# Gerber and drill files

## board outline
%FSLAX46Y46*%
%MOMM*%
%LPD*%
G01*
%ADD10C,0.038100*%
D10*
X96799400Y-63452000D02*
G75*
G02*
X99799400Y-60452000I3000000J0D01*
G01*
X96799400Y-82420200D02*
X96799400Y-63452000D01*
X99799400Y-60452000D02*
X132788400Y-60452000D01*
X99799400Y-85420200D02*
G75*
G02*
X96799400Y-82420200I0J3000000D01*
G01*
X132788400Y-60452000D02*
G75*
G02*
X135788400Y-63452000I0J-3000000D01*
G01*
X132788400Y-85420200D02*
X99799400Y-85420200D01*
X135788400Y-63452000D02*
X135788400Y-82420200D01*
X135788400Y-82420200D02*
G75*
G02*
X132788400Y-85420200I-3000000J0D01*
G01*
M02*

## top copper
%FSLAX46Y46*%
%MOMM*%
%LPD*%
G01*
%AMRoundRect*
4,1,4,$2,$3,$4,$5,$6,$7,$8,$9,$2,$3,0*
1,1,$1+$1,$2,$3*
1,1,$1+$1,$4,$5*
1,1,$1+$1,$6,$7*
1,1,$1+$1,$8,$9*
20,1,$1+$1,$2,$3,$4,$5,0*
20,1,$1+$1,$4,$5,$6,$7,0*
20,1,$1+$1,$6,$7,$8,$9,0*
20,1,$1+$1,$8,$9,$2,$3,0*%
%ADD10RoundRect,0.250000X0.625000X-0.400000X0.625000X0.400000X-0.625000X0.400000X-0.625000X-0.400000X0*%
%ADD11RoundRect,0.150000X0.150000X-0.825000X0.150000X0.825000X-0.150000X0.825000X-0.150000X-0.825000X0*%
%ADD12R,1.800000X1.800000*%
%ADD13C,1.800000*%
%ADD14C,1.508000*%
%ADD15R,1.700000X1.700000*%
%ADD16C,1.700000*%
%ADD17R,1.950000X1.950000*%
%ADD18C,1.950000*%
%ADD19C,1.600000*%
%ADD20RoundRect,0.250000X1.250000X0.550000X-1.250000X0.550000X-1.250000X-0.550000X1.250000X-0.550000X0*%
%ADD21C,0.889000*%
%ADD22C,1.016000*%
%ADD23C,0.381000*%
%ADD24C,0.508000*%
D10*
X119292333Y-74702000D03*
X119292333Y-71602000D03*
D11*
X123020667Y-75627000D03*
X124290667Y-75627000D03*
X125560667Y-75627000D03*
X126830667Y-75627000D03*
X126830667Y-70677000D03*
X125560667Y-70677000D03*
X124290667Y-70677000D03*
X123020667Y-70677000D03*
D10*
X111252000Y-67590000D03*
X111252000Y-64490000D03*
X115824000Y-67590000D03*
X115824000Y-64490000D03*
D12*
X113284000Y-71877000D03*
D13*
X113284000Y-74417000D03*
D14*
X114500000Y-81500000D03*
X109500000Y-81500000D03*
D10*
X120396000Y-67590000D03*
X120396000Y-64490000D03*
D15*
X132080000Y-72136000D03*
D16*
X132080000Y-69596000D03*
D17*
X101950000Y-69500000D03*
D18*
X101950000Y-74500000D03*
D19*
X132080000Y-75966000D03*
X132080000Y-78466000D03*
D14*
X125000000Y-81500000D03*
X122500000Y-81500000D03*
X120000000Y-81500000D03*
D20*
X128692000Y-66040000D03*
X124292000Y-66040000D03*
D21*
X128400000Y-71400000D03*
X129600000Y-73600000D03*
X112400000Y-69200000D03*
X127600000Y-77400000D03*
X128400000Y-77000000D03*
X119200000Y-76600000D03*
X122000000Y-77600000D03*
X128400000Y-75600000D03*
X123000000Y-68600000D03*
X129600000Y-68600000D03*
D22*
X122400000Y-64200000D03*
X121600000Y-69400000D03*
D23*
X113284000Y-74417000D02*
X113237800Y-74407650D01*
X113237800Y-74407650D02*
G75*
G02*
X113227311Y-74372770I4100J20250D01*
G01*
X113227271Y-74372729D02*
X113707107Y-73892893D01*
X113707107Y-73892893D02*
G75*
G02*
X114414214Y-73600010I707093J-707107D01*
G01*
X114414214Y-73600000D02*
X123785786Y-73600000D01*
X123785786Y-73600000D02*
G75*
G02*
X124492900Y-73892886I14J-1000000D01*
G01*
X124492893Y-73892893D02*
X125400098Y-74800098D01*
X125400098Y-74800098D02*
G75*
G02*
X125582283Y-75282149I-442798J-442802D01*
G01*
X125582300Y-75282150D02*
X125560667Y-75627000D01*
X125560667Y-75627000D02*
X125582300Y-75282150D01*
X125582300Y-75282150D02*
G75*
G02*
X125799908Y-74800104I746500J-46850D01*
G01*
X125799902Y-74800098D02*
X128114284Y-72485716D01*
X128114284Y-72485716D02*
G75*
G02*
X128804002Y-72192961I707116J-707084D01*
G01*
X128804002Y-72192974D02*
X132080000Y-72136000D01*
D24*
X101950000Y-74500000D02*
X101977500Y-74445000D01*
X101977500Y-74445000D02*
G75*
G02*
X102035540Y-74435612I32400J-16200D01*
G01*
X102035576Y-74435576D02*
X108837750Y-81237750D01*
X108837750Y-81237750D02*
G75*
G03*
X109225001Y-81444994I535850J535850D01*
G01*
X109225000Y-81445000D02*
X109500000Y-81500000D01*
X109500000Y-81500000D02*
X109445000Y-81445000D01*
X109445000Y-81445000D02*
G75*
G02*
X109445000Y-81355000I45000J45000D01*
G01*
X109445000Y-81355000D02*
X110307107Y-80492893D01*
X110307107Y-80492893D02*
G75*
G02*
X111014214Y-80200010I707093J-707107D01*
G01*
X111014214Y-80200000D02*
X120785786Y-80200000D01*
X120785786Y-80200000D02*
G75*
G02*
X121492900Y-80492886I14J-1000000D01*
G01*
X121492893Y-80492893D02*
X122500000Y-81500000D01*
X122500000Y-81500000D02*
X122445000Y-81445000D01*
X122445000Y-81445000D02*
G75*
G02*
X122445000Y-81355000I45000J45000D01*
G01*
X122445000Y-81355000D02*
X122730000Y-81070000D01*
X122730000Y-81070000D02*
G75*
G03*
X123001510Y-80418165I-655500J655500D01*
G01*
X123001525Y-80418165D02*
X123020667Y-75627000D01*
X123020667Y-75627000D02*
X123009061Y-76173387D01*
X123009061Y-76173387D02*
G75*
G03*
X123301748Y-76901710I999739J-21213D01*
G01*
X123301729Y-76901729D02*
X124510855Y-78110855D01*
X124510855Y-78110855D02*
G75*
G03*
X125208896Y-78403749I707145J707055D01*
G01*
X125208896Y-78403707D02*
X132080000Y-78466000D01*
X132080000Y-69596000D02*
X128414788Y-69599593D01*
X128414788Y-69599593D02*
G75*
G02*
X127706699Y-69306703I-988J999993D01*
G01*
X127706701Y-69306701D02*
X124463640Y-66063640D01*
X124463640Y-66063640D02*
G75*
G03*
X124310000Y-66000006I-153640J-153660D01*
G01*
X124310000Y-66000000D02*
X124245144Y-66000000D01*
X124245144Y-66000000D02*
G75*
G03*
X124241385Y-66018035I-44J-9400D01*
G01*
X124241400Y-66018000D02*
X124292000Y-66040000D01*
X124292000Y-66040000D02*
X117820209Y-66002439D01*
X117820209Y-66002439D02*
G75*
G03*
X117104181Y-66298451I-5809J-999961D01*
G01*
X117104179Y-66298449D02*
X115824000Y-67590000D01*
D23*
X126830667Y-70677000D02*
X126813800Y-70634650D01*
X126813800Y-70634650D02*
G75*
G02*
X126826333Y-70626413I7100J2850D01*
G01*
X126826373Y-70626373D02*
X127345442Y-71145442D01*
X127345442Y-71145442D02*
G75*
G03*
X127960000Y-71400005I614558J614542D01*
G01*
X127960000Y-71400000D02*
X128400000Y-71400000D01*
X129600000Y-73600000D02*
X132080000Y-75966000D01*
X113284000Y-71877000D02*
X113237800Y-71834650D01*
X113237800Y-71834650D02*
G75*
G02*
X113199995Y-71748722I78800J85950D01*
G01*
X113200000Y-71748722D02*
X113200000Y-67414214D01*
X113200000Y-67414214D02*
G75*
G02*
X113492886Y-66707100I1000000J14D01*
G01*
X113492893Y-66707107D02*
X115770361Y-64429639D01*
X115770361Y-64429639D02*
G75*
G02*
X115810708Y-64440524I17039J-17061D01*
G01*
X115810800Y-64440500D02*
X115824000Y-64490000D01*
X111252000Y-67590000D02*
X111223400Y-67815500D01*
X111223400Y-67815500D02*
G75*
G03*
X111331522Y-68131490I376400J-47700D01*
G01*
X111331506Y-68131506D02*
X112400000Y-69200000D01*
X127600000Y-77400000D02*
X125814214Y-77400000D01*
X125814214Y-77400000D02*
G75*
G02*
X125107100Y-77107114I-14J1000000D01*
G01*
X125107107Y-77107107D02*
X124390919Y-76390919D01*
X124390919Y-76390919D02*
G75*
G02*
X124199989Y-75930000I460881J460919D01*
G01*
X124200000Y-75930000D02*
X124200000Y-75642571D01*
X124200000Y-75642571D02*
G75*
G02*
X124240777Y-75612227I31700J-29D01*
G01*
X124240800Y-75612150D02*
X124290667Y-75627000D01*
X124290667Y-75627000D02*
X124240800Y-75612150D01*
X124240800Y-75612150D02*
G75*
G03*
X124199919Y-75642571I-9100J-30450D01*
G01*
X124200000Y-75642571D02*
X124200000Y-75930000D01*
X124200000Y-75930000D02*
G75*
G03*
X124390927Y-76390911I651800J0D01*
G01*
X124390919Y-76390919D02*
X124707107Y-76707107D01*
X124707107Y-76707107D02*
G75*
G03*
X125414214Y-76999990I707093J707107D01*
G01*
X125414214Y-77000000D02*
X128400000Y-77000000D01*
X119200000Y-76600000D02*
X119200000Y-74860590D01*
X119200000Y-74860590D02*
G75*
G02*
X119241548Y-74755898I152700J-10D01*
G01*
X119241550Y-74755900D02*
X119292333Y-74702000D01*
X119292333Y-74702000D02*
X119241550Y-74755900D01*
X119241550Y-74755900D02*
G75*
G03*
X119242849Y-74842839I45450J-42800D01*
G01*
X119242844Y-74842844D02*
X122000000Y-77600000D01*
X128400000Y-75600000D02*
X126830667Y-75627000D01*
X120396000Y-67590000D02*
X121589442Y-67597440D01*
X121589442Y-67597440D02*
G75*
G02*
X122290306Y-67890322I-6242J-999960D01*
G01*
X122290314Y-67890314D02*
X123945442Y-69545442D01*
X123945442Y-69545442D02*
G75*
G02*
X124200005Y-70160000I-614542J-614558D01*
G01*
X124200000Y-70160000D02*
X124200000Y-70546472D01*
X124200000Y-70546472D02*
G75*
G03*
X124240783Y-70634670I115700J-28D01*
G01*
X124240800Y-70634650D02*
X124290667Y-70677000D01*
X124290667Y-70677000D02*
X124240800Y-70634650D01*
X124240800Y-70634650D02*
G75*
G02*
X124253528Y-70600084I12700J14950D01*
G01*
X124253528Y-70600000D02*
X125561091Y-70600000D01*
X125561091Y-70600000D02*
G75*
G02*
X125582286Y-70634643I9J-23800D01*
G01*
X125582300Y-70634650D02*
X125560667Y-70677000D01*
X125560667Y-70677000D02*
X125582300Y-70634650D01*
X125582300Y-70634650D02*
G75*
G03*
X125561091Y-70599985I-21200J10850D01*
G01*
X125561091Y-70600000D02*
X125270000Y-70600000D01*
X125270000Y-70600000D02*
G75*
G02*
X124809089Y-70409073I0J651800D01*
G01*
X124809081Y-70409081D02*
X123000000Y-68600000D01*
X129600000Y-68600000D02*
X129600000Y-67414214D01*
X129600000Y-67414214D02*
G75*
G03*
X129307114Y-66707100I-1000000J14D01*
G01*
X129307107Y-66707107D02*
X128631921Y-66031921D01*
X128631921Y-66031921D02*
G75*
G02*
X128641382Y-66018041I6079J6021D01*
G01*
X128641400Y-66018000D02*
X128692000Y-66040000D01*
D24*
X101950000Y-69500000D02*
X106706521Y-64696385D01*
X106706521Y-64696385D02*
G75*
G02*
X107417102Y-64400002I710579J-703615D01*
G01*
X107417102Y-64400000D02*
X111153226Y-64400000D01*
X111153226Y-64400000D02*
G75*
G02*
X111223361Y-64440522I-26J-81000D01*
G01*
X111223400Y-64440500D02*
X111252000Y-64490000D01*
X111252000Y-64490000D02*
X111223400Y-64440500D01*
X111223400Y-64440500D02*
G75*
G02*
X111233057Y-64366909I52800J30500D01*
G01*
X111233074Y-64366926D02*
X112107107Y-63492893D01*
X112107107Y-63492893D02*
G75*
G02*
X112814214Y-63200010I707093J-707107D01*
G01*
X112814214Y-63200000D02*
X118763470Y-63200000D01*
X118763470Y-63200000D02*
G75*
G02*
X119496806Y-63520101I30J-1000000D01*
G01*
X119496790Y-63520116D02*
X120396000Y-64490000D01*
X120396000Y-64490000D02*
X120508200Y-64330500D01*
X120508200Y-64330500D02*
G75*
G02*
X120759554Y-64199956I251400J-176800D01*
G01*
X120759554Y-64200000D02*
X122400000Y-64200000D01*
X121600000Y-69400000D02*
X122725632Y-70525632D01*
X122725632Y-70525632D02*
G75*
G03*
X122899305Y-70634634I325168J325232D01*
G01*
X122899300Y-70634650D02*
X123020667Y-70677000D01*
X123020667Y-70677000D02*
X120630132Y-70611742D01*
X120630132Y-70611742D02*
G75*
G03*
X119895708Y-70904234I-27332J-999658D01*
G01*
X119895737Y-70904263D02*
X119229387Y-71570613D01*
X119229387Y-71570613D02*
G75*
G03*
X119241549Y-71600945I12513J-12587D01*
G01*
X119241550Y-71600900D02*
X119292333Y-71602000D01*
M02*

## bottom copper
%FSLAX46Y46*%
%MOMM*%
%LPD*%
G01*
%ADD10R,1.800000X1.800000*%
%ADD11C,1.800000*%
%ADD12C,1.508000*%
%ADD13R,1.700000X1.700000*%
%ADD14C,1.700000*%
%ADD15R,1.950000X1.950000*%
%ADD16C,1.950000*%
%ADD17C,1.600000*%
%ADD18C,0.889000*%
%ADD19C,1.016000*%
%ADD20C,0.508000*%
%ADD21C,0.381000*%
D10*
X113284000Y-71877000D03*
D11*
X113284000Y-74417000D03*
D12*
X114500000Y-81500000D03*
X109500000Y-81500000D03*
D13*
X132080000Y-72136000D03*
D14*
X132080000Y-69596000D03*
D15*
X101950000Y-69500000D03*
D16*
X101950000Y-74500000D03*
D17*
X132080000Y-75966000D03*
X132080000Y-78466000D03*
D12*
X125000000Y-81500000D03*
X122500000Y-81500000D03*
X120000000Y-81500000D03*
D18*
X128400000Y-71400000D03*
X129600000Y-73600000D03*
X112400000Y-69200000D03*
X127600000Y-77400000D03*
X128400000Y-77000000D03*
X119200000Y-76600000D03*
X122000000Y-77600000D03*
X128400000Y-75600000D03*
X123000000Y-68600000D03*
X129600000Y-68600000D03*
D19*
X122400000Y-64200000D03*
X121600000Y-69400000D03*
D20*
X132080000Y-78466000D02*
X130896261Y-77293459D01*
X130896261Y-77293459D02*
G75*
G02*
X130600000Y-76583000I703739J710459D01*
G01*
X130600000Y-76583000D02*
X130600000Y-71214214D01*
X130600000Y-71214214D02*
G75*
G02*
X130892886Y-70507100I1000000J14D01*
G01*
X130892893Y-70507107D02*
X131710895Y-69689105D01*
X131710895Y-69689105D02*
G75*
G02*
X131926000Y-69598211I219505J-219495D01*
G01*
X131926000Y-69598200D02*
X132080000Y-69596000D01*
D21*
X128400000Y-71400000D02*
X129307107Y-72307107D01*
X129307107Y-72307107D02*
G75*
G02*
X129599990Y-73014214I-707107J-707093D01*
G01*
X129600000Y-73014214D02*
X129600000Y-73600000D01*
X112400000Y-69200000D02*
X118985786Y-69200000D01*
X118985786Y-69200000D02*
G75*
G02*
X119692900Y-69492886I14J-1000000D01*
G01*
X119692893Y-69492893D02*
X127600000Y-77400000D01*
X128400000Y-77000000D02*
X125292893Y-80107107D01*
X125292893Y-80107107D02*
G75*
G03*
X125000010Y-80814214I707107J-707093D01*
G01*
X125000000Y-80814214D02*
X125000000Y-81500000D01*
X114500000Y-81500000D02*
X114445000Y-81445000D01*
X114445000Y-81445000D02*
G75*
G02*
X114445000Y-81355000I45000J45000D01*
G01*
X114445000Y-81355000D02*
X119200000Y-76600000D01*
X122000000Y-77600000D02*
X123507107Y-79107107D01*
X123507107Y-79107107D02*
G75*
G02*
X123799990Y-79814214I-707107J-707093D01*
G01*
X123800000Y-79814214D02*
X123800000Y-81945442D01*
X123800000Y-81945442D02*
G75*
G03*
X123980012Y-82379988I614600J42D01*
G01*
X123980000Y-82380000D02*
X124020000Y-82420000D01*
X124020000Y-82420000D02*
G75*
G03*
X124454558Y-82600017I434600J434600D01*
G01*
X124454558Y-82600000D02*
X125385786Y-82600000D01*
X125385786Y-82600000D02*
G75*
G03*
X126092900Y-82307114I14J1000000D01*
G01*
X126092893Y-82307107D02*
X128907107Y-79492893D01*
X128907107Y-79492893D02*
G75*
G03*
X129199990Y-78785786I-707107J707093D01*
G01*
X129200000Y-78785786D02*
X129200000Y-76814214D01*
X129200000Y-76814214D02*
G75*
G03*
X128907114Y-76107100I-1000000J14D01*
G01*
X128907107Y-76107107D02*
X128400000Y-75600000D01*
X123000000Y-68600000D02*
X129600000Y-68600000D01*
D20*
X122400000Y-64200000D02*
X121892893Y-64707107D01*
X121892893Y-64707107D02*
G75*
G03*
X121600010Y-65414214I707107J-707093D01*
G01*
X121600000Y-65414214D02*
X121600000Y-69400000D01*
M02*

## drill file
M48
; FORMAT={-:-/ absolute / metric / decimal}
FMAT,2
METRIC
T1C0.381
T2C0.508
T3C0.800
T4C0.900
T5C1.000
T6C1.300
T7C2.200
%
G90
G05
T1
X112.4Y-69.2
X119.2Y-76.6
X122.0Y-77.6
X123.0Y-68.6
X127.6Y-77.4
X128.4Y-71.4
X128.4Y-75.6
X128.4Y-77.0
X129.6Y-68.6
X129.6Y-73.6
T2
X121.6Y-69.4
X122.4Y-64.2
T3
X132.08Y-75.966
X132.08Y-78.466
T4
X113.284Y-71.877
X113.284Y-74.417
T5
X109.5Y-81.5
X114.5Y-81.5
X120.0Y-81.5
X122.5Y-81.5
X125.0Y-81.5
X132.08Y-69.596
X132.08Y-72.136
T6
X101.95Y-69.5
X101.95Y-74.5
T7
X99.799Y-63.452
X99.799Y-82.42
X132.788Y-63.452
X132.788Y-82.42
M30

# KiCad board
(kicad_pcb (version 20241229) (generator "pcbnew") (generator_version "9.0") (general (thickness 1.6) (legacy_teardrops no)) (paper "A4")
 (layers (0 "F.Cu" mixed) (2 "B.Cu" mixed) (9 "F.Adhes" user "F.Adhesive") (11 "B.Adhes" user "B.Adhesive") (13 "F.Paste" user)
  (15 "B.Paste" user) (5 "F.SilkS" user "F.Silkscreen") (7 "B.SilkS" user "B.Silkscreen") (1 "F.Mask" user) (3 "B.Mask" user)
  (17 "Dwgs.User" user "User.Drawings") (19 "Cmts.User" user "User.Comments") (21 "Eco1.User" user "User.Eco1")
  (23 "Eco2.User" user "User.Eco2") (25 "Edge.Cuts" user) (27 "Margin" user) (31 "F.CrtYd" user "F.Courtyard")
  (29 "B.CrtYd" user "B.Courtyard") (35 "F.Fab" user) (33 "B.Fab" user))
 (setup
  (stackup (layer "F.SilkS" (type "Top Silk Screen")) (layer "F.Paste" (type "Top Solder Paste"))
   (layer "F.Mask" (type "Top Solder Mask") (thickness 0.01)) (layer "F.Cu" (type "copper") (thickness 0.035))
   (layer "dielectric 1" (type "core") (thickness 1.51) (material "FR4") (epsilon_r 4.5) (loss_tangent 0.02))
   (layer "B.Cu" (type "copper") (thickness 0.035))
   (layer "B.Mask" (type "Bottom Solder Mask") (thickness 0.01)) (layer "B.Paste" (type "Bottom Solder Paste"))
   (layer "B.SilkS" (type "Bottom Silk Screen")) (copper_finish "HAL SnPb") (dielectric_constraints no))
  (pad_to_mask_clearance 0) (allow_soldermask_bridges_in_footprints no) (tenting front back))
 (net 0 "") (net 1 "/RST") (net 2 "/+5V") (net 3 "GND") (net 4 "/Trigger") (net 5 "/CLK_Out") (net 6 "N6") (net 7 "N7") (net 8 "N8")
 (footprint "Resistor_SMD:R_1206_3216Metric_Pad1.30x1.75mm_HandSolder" (layer "F.Cu") (at 119.292333 73.152 90)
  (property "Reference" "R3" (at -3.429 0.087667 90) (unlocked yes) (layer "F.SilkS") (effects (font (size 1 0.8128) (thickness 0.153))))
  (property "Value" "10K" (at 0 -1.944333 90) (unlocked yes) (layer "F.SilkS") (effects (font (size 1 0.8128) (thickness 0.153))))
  (pad "1" smd roundrect (at -1.55 0 90) (size 1.3 1.75) (layers "F.Cu" "F.Mask" "F.Paste") (roundrect_rratio 0.192308) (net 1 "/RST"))
  (pad "2" smd roundrect (at 1.55 0 90) (size 1.3 1.75) (layers "F.Cu" "F.Mask" "F.Paste") (roundrect_rratio 0.192308) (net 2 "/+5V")))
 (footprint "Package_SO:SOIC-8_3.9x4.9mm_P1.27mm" (layer "F.Cu") (at 124.925667 73.152 90)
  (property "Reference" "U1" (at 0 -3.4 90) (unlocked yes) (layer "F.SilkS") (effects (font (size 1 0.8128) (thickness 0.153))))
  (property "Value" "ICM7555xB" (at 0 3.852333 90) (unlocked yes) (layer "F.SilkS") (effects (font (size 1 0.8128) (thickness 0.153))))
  (pad "1" smd roundrect (at -2.475 -1.905 90) (size 1.95 0.6) (layers "F.Cu" "F.Mask" "F.Paste") (roundrect_rratio 0.25) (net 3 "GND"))
  (pad "2" smd roundrect (at -2.475 -0.635 90) (size 1.95 0.6) (layers "F.Cu" "F.Mask" "F.Paste") (roundrect_rratio 0.25) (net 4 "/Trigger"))
  (pad "3" smd roundrect (at -2.475 0.635 90) (size 1.95 0.6) (layers "F.Cu" "F.Mask" "F.Paste") (roundrect_rratio 0.25) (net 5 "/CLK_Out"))
  (pad "4" smd roundrect (at -2.475 1.905 90) (size 1.95 0.6) (layers "F.Cu" "F.Mask" "F.Paste") (roundrect_rratio 0.25) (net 1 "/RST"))
  (pad "5" smd roundrect (at 2.475 1.905 90) (size 1.95 0.6) (layers "F.Cu" "F.Mask" "F.Paste") (roundrect_rratio 0.25) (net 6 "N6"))
  (pad "6" smd roundrect (at 2.475 0.635 90) (size 1.95 0.6) (layers "F.Cu" "F.Mask" "F.Paste") (roundrect_rratio 0.25) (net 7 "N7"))
  (pad "7" smd roundrect (at 2.475 -0.635 90) (size 1.95 0.6) (layers "F.Cu" "F.Mask" "F.Paste") (roundrect_rratio 0.25) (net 7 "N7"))
  (pad "8" smd roundrect (at 2.475 -1.905 90) (size 1.95 0.6) (layers "F.Cu" "F.Mask" "F.Paste") (roundrect_rratio 0.25) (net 2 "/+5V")))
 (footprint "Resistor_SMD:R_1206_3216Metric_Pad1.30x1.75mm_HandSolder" (layer "F.Cu") (at 111.252 66.04 90)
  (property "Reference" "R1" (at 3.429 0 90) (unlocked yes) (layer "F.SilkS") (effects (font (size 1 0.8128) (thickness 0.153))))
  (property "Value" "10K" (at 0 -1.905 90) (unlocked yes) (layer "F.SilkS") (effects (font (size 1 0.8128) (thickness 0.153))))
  (pad "1" smd roundrect (at -1.55 0 90) (size 1.3 1.75) (layers "F.Cu" "F.Mask" "F.Paste") (roundrect_rratio 0.192308) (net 4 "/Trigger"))
  (pad "2" smd roundrect (at 1.55 0 90) (size 1.3 1.75) (layers "F.Cu" "F.Mask" "F.Paste") (roundrect_rratio 0.192308) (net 2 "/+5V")))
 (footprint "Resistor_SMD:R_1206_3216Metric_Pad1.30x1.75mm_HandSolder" (layer "F.Cu") (at 115.824 66.04 90)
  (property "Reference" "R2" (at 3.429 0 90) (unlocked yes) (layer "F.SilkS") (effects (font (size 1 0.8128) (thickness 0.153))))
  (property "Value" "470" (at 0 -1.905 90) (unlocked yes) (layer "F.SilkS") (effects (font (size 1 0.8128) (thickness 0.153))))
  (pad "1" smd roundrect (at -1.55 0 90) (size 1.3 1.75) (layers "F.Cu" "F.Mask" "F.Paste") (roundrect_rratio 0.192308) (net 3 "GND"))
  (pad "2" smd roundrect (at 1.55 0 90) (size 1.3 1.75) (layers "F.Cu" "F.Mask" "F.Paste") (roundrect_rratio 0.192308) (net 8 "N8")))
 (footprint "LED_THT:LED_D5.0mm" (layer "F.Cu") (at 113.284 71.877 -90)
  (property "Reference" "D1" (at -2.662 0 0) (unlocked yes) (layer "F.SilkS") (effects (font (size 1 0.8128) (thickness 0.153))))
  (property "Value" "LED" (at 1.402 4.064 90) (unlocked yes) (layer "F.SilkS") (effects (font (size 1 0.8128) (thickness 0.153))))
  (pad "1" thru_hole rect (at 0 0 270) (size 1.8 1.8) (drill 0.9) (layers "*.Cu" "*.Mask") (remove_unused_layers no) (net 8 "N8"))
  (pad "2" thru_hole circle (at 2.54 0 270) (size 1.8 1.8) (drill 0.9) (layers "*.Cu" "*.Mask") (remove_unused_layers no) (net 5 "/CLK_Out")))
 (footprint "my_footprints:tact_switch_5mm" (layer "F.Cu") (at 112 81.5 180)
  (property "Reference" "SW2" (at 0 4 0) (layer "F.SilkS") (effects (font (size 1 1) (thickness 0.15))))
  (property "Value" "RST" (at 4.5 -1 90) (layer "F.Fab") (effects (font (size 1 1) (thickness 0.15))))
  (pad "1" thru_hole circle (at -2.5 0 180) (size 1.508 1.508) (drill 1) (layers "*.Cu" "*.Mask") (remove_unused_layers no) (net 1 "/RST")
   (solder_mask_margin 0.102))
  (pad "2" thru_hole circle (at 2.5 0 180) (size 1.508 1.508) (drill 1) (layers "*.Cu" "*.Mask") (remove_unused_layers no) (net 3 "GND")
   (solder_mask_margin 0.102)))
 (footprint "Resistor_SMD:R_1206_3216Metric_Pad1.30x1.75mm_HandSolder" (layer "F.Cu") (at 120.396 66.04 90)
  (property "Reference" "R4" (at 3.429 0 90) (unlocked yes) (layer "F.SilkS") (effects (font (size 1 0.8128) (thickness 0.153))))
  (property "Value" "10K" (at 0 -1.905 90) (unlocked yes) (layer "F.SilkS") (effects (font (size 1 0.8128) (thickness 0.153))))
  (pad "1" smd roundrect (at -1.55 0 90) (size 1.3 1.75) (layers "F.Cu" "F.Mask" "F.Paste") (roundrect_rratio 0.192308) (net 7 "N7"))
  (pad "2" smd roundrect (at 1.55 0 90) (size 1.3 1.75) (layers "F.Cu" "F.Mask" "F.Paste") (roundrect_rratio 0.192308) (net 2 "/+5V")))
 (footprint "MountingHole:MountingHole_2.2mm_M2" (layer "F.Cu") (at 99.7994 63.452)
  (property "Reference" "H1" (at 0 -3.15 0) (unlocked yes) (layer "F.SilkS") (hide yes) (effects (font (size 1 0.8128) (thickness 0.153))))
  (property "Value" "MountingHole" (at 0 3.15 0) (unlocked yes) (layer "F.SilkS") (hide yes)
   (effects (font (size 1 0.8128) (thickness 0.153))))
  (pad "" np_thru_hole circle (at 0 0) (size 2.2 2.2) (drill 2.2) (layers "*.Cu" "*.Mask")))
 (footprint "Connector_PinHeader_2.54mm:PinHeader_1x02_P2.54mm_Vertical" (layer "F.Cu") (at 132.08 72.136 180)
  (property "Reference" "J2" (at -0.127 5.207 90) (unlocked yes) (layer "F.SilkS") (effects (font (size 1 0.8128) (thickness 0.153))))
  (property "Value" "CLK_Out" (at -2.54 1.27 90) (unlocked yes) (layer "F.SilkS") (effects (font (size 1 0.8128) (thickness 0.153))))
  (pad "1" thru_hole rect (at 0 0 180) (size 1.7 1.7) (drill 1) (layers "*.Cu" "*.Mask") (remove_unused_layers no) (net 5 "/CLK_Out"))
  (pad "2" thru_hole circle (at 0 2.54 180) (size 1.7 1.7) (drill 1) (layers "*.Cu" "*.Mask") (remove_unused_layers no) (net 3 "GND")))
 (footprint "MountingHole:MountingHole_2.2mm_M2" (layer "F.Cu") (at 132.7884 82.4202)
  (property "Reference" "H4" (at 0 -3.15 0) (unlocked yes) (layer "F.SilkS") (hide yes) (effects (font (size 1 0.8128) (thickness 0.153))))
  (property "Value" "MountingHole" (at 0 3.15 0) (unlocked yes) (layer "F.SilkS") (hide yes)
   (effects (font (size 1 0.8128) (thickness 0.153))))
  (pad "" np_thru_hole circle (at 0 0) (size 2.2 2.2) (drill 2.2) (layers "*.Cu" "*.Mask")))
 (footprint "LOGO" (layer "F.Cu") (at 105.5 63.5)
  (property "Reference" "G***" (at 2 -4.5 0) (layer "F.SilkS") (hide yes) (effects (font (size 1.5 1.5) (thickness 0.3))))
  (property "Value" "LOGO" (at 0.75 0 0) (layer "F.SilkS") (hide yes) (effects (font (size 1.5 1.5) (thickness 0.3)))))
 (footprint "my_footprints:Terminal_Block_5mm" (layer "F.Cu") (at 101.95 72 -90)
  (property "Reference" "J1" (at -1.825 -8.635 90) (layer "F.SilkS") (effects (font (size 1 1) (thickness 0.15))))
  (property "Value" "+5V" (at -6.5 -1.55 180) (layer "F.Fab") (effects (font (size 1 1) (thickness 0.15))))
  (pad "1" thru_hole rect (at -2.5 0 270) (size 1.95 1.95) (drill 1.3) (layers "*.Cu" "*.Mask") (remove_unused_layers no) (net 2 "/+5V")
   (solder_mask_margin 0.102))
  (pad "2" thru_hole circle (at 2.5 0 270) (size 1.95 1.95) (drill 1.3) (layers "*.Cu" "*.Mask") (remove_unused_layers no) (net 3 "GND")
   (solder_mask_margin 0.102)))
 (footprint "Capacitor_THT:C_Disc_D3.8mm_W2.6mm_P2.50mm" (layer "F.Cu") (at 132.08 75.966 -90)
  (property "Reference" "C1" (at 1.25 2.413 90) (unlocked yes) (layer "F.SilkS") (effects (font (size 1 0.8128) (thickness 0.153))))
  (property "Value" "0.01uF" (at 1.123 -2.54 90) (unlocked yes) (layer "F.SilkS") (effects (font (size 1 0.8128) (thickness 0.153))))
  (pad "1" thru_hole circle (at 0 0 270) (size 1.6 1.6) (drill 0.8) (layers "*.Cu" "*.Mask") (remove_unused_layers no) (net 6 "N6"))
  (pad "2" thru_hole circle (at 2.5 0 270) (size 1.6 1.6) (drill 0.8) (layers "*.Cu" "*.Mask") (remove_unused_layers no) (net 3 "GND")))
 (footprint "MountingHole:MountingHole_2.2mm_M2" (layer "F.Cu") (at 132.7884 63.452)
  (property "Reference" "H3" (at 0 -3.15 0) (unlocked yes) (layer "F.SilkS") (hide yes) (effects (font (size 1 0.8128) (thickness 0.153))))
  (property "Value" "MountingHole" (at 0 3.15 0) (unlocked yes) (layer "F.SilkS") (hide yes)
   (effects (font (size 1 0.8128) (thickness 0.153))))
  (pad "" np_thru_hole circle (at 0 0) (size 2.2 2.2) (drill 2.2) (layers "*.Cu" "*.Mask")))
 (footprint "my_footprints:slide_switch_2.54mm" (layer "F.Cu") (at 122.5 81.5 180)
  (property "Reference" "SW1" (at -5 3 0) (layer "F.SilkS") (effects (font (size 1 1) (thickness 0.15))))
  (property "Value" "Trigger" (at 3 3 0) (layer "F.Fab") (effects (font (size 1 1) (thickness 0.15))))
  (pad "1" thru_hole circle (at -2.5 0 180) (size 1.508 1.508) (drill 1) (layers "*.Cu" "*.Mask") (remove_unused_layers no)
   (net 4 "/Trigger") (solder_mask_margin 0.102))
  (pad "2" thru_hole circle (at 0 0 180) (size 1.508 1.508) (drill 1) (layers "*.Cu" "*.Mask") (remove_unused_layers no) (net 3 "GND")
   (solder_mask_margin 0.102))
  (pad "3" thru_hole circle (at 2.5 0 180) (size 1.508 1.508) (drill 1) (layers "*.Cu" "*.Mask") (remove_unused_layers no)
   (solder_mask_margin 0.102)))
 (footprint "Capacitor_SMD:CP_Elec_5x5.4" (layer "F.Cu") (at 126.492 66.04 180)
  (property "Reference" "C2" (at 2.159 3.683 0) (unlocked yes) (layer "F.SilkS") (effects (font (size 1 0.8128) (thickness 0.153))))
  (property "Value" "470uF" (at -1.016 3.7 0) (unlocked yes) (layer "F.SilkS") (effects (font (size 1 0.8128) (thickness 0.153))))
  (pad "1" smd roundrect (at -2.2 0 180) (size 3 1.6) (layers "F.Cu" "F.Mask" "F.Paste") (roundrect_rratio 0.15625) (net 7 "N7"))
  (pad "2" smd roundrect (at 2.2 0 180) (size 3 1.6) (layers "F.Cu" "F.Mask" "F.Paste") (roundrect_rratio 0.15625) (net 3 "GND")))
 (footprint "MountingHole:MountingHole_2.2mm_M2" (layer "F.Cu") (at 99.7994 82.4202)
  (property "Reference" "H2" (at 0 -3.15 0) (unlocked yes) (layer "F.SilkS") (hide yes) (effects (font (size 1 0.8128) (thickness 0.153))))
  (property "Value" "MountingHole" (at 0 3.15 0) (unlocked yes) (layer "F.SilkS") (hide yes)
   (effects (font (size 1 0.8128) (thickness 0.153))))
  (pad "" np_thru_hole circle (at 0 0) (size 2.2 2.2) (drill 2.2) (layers "*.Cu" "*.Mask")))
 (gr_arc (start 96.7994 63.452) (mid 97.67808 61.33068) (end 99.7994 60.452) (stroke (width 0.0381) (type default)) (layer "Edge.Cuts"))
 (gr_line (start 96.7994 82.4202) (end 96.7994 63.452) (stroke (width 0.0381) (type default)) (layer "Edge.Cuts"))
 (gr_line (start 99.7994 60.452) (end 132.7884 60.452) (stroke (width 0.0381) (type default)) (layer "Edge.Cuts"))
 (gr_arc (start 99.7994 85.4202) (mid 97.67808 84.54152) (end 96.7994 82.4202) (stroke (width 0.0381) (type default)) (layer "Edge.Cuts"))
 (gr_arc (start 132.7884 60.452) (mid 134.90972 61.33068) (end 135.7884 63.452) (stroke (width 0.0381) (type default)) (layer "Edge.Cuts"))
 (gr_line (start 132.7884 85.4202) (end 99.7994 85.4202) (stroke (width 0.0381) (type default)) (layer "Edge.Cuts"))
 (gr_line (start 135.7884 63.452) (end 135.7884 82.4202) (stroke (width 0.0381) (type default)) (layer "Edge.Cuts"))
 (gr_arc (start 135.7884 82.4202) (mid 134.90972 84.54152) (end 132.7884 85.4202) (stroke (width 0.0381) (type default)) (layer "Edge.Cuts"))
 (segment (start 113.284000 74.417000) (end 113.237800 74.407650) (width 0.381000) (layer "F.Cu") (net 5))
 (arc (start 113.237800 74.407650) (mid 113.222090 74.393339) (end 113.227271 74.372729) (width 0.381000) (layer "F.Cu") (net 5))
 (segment (start 113.227271 74.372729) (end 113.707107 73.892893) (width 0.381000) (layer "F.Cu") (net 5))
 (arc (start 113.707107 73.892893) (mid 114.031530 73.676120) (end 114.414214 73.600000) (width 0.381000) (layer "F.Cu") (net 5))
 (segment (start 114.414214 73.600000) (end 123.785786 73.600000) (width 0.381000) (layer "F.Cu") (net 5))
 (arc (start 123.785786 73.600000) (mid 124.168470 73.676120) (end 124.492893 73.892893) (width 0.381000) (layer "F.Cu") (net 5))
 (segment (start 124.492893 73.892893) (end 125.400098 74.800098) (width 0.381000) (layer "F.Cu") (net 5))
 (arc (start 125.400098 74.800098) (mid 125.543079 75.021515) (end 125.582300 75.282150) (width 0.381000) (layer "F.Cu") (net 5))
 (segment (start 125.582300 75.282150) (end 125.560667 75.627000) (width 0.381000) (layer "F.Cu") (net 5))
 (segment (start 125.560667 75.627000) (end 125.582300 75.282150) (width 0.381000) (layer "F.Cu") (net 5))
 (arc (start 125.582300 75.282150) (mid 125.647071 75.021248) (end 125.799902 74.800098) (width 0.381000) (layer "F.Cu") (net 5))
 (segment (start 125.799902 74.800098) (end 128.114284 72.485716) (width 0.381000) (layer "F.Cu") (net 5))
 (arc (start 128.114284 72.485716) (mid 128.430689 72.272305) (end 128.804002 72.192974) (width 0.381000) (layer "F.Cu") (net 5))
 (segment (start 128.804002 72.192974) (end 132.080000 72.136000) (width 0.381000) (layer "F.Cu") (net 5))
 (segment (start 101.950000 74.500000) (end 101.977500 74.445000) (width 0.508000) (layer "F.Cu") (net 3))
 (arc (start 101.977500 74.445000) (mid 102.004126 74.425423) (end 102.035576 74.435576) (width 0.508000) (layer "F.Cu") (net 3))
 (segment (start 102.035576 74.435576) (end 108.837750 81.237750) (width 0.508000) (layer "F.Cu") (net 3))
 (arc (start 108.837750 81.237750) (mid 109.016031 81.370045) (end 109.225000 81.445000) (width 0.508000) (layer "F.Cu") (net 3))
 (segment (start 109.225000 81.445000) (end 109.500000 81.500000) (width 0.508000) (layer "F.Cu") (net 3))
 (segment (start 109.500000 81.500000) (end 109.445000 81.445000) (width 0.508000) (layer "F.Cu") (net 3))
 (arc (start 109.445000 81.445000) (mid 109.426360 81.400000) (end 109.445000 81.355000) (width 0.508000) (layer "F.Cu") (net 3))
 (segment (start 109.445000 81.355000) (end 110.307107 80.492893) (width 0.508000) (layer "F.Cu") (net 3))
 (arc (start 110.307107 80.492893) (mid 110.631530 80.276120) (end 111.014214 80.200000) (width 0.508000) (layer "F.Cu") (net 3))
 (segment (start 111.014214 80.200000) (end 120.785786 80.200000) (width 0.508000) (layer "F.Cu") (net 3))
 (arc (start 120.785786 80.200000) (mid 121.168470 80.276120) (end 121.492893 80.492893) (width 0.508000) (layer "F.Cu") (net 3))
 (segment (start 121.492893 80.492893) (end 122.500000 81.500000) (width 0.508000) (layer "F.Cu") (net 3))
 (segment (start 122.500000 81.500000) (end 122.445000 81.445000) (width 0.508000) (layer "F.Cu") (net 3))
 (arc (start 122.445000 81.445000) (mid 122.426360 81.400000) (end 122.445000 81.355000) (width 0.508000) (layer "F.Cu") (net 3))
 (segment (start 122.445000 81.355000) (end 122.730000 81.070000) (width 0.508000) (layer "F.Cu") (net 3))
 (arc (start 122.730000 81.070000) (mid 122.930253 80.770947) (end 123.001525 80.418165) (width 0.508000) (layer "F.Cu") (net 3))
 (segment (start 123.001525 80.418165) (end 123.020667 75.627000) (width 0.508000) (layer "F.Cu") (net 3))
 (segment (start 123.020667 75.627000) (end 123.009061 76.173387) (width 0.508000) (layer "F.Cu") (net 3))
 (arc (start 123.009061 76.173387) (mid 123.080945 76.567474) (end 123.301729 76.901729) (width 0.508000) (layer "F.Cu") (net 3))
 (segment (start 123.301729 76.901729) (end 124.510855 78.110855) (width 0.508000) (layer "F.Cu") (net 3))
 (arc (start 124.510855 78.110855) (mid 124.831094 78.325884) (end 125.208896 78.403707) (width 0.508000) (layer "F.Cu") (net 3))
 (segment (start 125.208896 78.403707) (end 132.080000 78.466000) (width 0.508000) (layer "F.Cu") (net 3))
 (segment (start 132.080000 78.466000) (end 130.896261 77.293459) (width 0.508000) (layer "B.Cu") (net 3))
 (arc (start 130.896261 77.293459) (mid 130.677032 76.967877) (end 130.600000 76.583000) (width 0.508000) (layer "B.Cu") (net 3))
 (segment (start 130.600000 76.583000) (end 130.600000 71.214214) (width 0.508000) (layer "B.Cu") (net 3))
 (arc (start 130.600000 71.214214) (mid 130.676120 70.831530) (end 130.892893 70.507107) (width 0.508000) (layer "B.Cu") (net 3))
 (segment (start 130.892893 70.507107) (end 131.710895 69.689105) (width 0.508000) (layer "B.Cu") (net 3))
 (arc (start 131.710895 69.689105) (mid 131.809575 69.622658) (end 131.926000 69.598200) (width 0.508000) (layer "B.Cu") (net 3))
 (segment (start 131.926000 69.598200) (end 132.080000 69.596000) (width 0.508000) (layer "B.Cu") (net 3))
 (segment (start 132.080000 69.596000) (end 128.414788 69.599593) (width 0.508000) (layer "F.Cu") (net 3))
 (arc (start 128.414788 69.599593) (mid 128.031577 69.523661) (end 127.706701 69.306701) (width 0.508000) (layer "F.Cu") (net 3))
 (segment (start 127.706701 69.306701) (end 124.463640 66.063640) (width 0.508000) (layer "F.Cu") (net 3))
 (arc (start 124.463640 66.063640) (mid 124.393149 66.016539) (end 124.310000 66.000000) (width 0.508000) (layer "F.Cu") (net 3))
 (segment (start 124.310000 66.000000) (end 124.245144 66.000000) (width 0.508000) (layer "F.Cu") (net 3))
 (arc (start 124.245144 66.000000) (mid 124.235951 66.007477) (end 124.241400 66.018000) (width 0.508000) (layer "F.Cu") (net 3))
 (segment (start 124.241400 66.018000) (end 124.292000 66.040000) (width 0.508000) (layer "F.Cu") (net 3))
 (segment (start 124.292000 66.040000) (end 117.820209 66.002439) (width 0.508000) (layer "F.Cu") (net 3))
 (arc (start 117.820209 66.002439) (mid 117.432361 66.078278) (end 117.104179 66.298449) (width 0.508000) (layer "F.Cu") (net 3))
 (segment (start 117.104179 66.298449) (end 115.824000 67.590000) (width 0.508000) (layer "F.Cu") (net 3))
 (segment (start 126.830667 70.677000) (end 126.813800 70.634650) (width 0.381000) (layer "F.Cu") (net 6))
 (arc (start 126.813800 70.634650) (mid 126.816714 70.625388) (end 126.826373 70.626373) (width 0.381000) (layer "F.Cu") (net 6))
 (segment (start 126.826373 70.626373) (end 127.345442 71.145442) (width 0.381000) (layer "F.Cu") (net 6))
 (arc (start 127.345442 71.145442) (mid 127.627403 71.333842) (end 127.960000 71.400000) (width 0.381000) (layer "F.Cu") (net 6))
 (segment (start 127.960000 71.400000) (end 128.400000 71.400000) (width 0.381000) (layer "F.Cu") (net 6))
 (segment (start 128.400000 71.400000) (end 129.307107 72.307107) (width 0.381000) (layer "B.Cu") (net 6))
 (arc (start 129.307107 72.307107) (mid 129.523880 72.631530) (end 129.600000 73.014214) (width 0.381000) (layer "B.Cu") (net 6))
 (segment (start 129.600000 73.014214) (end 129.600000 73.600000) (width 0.381000) (layer "B.Cu") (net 6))
 (segment (start 129.600000 73.600000) (end 132.080000 75.966000) (width 0.381000) (layer "F.Cu") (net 6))
 (segment (start 113.284000 71.877000) (end 113.237800 71.834650) (width 0.381000) (layer "F.Cu") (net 8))
 (arc (start 113.237800 71.834650) (mid 113.209868 71.795659) (end 113.200000 71.748722) (width 0.381000) (layer "F.Cu") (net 8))
 (segment (start 113.200000 71.748722) (end 113.200000 67.414214) (width 0.381000) (layer "F.Cu") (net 8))
 (arc (start 113.200000 67.414214) (mid 113.276120 67.031530) (end 113.492893 66.707107) (width 0.381000) (layer "F.Cu") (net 8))
 (segment (start 113.492893 66.707107) (end 115.770361 64.429639) (width 0.381000) (layer "F.Cu") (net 8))
 (arc (start 115.770361 64.429639) (mid 115.793718 64.423388) (end 115.810800 64.440500) (width 0.381000) (layer "F.Cu") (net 8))
 (segment (start 115.810800 64.440500) (end 115.824000 64.490000) (width 0.381000) (layer "F.Cu") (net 8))
 (segment (start 111.252000 67.590000) (end 111.223400 67.815500) (width 0.381000) (layer "F.Cu") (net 4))
 (arc (start 111.223400 67.815500) (mid 111.240810 67.986039) (end 111.331506 68.131506) (width 0.381000) (layer "F.Cu") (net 4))
 (segment (start 111.331506 68.131506) (end 112.400000 69.200000) (width 0.381000) (layer "F.Cu") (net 4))
 (segment (start 112.400000 69.200000) (end 118.985786 69.200000) (width 0.381000) (layer "B.Cu") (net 4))
 (arc (start 118.985786 69.200000) (mid 119.368470 69.276120) (end 119.692893 69.492893) (width 0.381000) (layer "B.Cu") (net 4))
 (segment (start 119.692893 69.492893) (end 127.600000 77.400000) (width 0.381000) (layer "B.Cu") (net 4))
 (segment (start 127.600000 77.400000) (end 125.814214 77.400000) (width 0.381000) (layer "F.Cu") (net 4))
 (arc (start 125.814214 77.400000) (mid 125.431530 77.323880) (end 125.107107 77.107107) (width 0.381000) (layer "F.Cu") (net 4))
 (segment (start 125.107107 77.107107) (end 124.390919 76.390919) (width 0.381000) (layer "F.Cu") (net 4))
 (arc (start 124.390919 76.390919) (mid 124.249618 76.179447) (end 124.200000 75.930000) (width 0.381000) (layer "F.Cu") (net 4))
 (segment (start 124.200000 75.930000) (end 124.200000 75.642571) (width 0.381000) (layer "F.Cu") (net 4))
 (arc (start 124.200000 75.642571) (mid 124.212768 75.617124) (end 124.240800 75.612150) (width 0.381000) (layer "F.Cu") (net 4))
 (segment (start 124.240800 75.612150) (end 124.290667 75.627000) (width 0.381000) (layer "F.Cu") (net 4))
 (segment (start 124.290667 75.627000) (end 124.240800 75.612150) (width 0.381000) (layer "F.Cu") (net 4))
 (arc (start 124.240800 75.612150) (mid 124.212768 75.617124) (end 124.200000 75.642571) (width 0.381000) (layer "F.Cu") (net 4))
 (segment (start 124.200000 75.642571) (end 124.200000 75.930000) (width 0.381000) (layer "F.Cu") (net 4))
 (arc (start 124.200000 75.930000) (mid 124.249618 76.179447) (end 124.390919 76.390919) (width 0.381000) (layer "F.Cu") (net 4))
 (segment (start 124.390919 76.390919) (end 124.707107 76.707107) (width 0.381000) (layer "F.Cu") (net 4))
 (arc (start 124.707107 76.707107) (mid 125.031530 76.923880) (end 125.414214 77.000000) (width 0.381000) (layer "F.Cu") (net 4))
 (segment (start 125.414214 77.000000) (end 128.400000 77.000000) (width 0.381000) (layer "F.Cu") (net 4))
 (segment (start 128.400000 77.000000) (end 125.292893 80.107107) (width 0.381000) (layer "B.Cu") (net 4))
 (arc (start 125.292893 80.107107) (mid 125.076120 80.431530) (end 125.000000 80.814214) (width 0.381000) (layer "B.Cu") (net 4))
 (segment (start 125.000000 80.814214) (end 125.000000 81.500000) (width 0.381000) (layer "B.Cu") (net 4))
 (segment (start 114.500000 81.500000) (end 114.445000 81.445000) (width 0.381000) (layer "B.Cu") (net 1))
 (arc (start 114.445000 81.445000) (mid 114.426360 81.400000) (end 114.445000 81.355000) (width 0.381000) (layer "B.Cu") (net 1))
 (segment (start 114.445000 81.355000) (end 119.200000 76.600000) (width 0.381000) (layer "B.Cu") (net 1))
 (segment (start 119.200000 76.600000) (end 119.200000 74.860590) (width 0.381000) (layer "F.Cu") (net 1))
 (arc (start 119.200000 74.860590) (mid 119.210767 74.804273) (end 119.241550 74.755900) (width 0.381000) (layer "F.Cu") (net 1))
 (segment (start 119.241550 74.755900) (end 119.292333 74.702000) (width 0.381000) (layer "F.Cu") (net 1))
 (segment (start 119.292333 74.702000) (end 119.241550 74.755900) (width 0.381000) (layer "F.Cu") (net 1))
 (arc (start 119.241550 74.755900) (mid 119.224568 74.799634) (end 119.242844 74.842844) (width 0.381000) (layer "F.Cu") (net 1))
 (segment (start 119.242844 74.842844) (end 122.000000 77.600000) (width 0.381000) (layer "F.Cu") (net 1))
 (segment (start 122.000000 77.600000) (end 123.507107 79.107107) (width 0.381000) (layer "B.Cu") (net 1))
 (arc (start 123.507107 79.107107) (mid 123.723880 79.431530) (end 123.800000 79.814214) (width 0.381000) (layer "B.Cu") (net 1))
 (segment (start 123.800000 79.814214) (end 123.800000 81.945442) (width 0.381000) (layer "B.Cu") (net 1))
 (arc (start 123.800000 81.945442) (mid 123.846780 82.180623) (end 123.980000 82.380000) (width 0.381000) (layer "B.Cu") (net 1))
 (segment (start 123.980000 82.380000) (end 124.020000 82.420000) (width 0.381000) (layer "B.Cu") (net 1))
 (arc (start 124.020000 82.420000) (mid 124.219377 82.553220) (end 124.454558 82.600000) (width 0.381000) (layer "B.Cu") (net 1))
 (segment (start 124.454558 82.600000) (end 125.385786 82.600000) (width 0.381000) (layer "B.Cu") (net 1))
 (arc (start 125.385786 82.600000) (mid 125.768470 82.523880) (end 126.092893 82.307107) (width 0.381000) (layer "B.Cu") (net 1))
 (segment (start 126.092893 82.307107) (end 128.907107 79.492893) (width 0.381000) (layer "B.Cu") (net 1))
 (arc (start 128.907107 79.492893) (mid 129.123880 79.168470) (end 129.200000 78.785786) (width 0.381000) (layer "B.Cu") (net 1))
 (segment (start 129.200000 78.785786) (end 129.200000 76.814214) (width 0.381000) (layer "B.Cu") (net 1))
 (arc (start 129.200000 76.814214) (mid 129.123880 76.431530) (end 128.907107 76.107107) (width 0.381000) (layer "B.Cu") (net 1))
 (segment (start 128.907107 76.107107) (end 128.400000 75.600000) (width 0.381000) (layer "B.Cu") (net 1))
 (segment (start 128.400000 75.600000) (end 126.830667 75.627000) (width 0.381000) (layer "F.Cu") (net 1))
 (segment (start 120.396000 67.590000) (end 121.589442 67.597440) (width 0.381000) (layer "F.Cu") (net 7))
 (arc (start 121.589442 67.597440) (mid 121.968769 67.674739) (end 122.290314 67.890314) (width 0.381000) (layer "F.Cu") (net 7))
 (segment (start 122.290314 67.890314) (end 123.945442 69.545442) (width 0.381000) (layer "F.Cu") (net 7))
 (arc (start 123.945442 69.545442) (mid 124.133842 69.827403) (end 124.200000 70.160000) (width 0.381000) (layer "F.Cu") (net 7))
 (segment (start 124.200000 70.160000) (end 124.200000 70.546472) (width 0.381000) (layer "F.Cu") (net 7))
 (arc (start 124.200000 70.546472) (mid 124.210694 70.595052) (end 124.240800 70.634650) (width 0.381000) (layer "F.Cu") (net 7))
 (segment (start 124.240800 70.634650) (end 124.290667 70.677000) (width 0.381000) (layer "F.Cu") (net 7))
 (segment (start 124.290667 70.677000) (end 124.240800 70.634650) (width 0.381000) (layer "F.Cu") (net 7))
 (arc (start 124.240800 70.634650) (mid 124.235071 70.612883) (end 124.253528 70.600000) (width 0.381000) (layer "F.Cu") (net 7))
 (segment (start 124.253528 70.600000) (end 125.561091 70.600000) (width 0.381000) (layer "F.Cu") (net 7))
 (arc (start 125.561091 70.600000) (mid 125.581404 70.611383) (end 125.582300 70.634650) (width 0.381000) (layer "F.Cu") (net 7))
 (segment (start 125.582300 70.634650) (end 125.560667 70.677000) (width 0.381000) (layer "F.Cu") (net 7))
 (segment (start 125.560667 70.677000) (end 125.582300 70.634650) (width 0.381000) (layer "F.Cu") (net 7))
 (arc (start 125.582300 70.634650) (mid 125.581404 70.611383) (end 125.561091 70.600000) (width 0.381000) (layer "F.Cu") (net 7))
 (segment (start 125.561091 70.600000) (end 125.270000 70.600000) (width 0.381000) (layer "F.Cu") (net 7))
 (arc (start 125.270000 70.600000) (mid 125.020553 70.550382) (end 124.809081 70.409081) (width 0.381000) (layer "F.Cu") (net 7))
 (segment (start 124.809081 70.409081) (end 123.000000 68.600000) (width 0.381000) (layer "F.Cu") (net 7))
 (segment (start 123.000000 68.600000) (end 129.600000 68.600000) (width 0.381000) (layer "B.Cu") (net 7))
 (segment (start 129.600000 68.600000) (end 129.600000 67.414214) (width 0.381000) (layer "F.Cu") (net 7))
 (arc (start 129.600000 67.414214) (mid 129.523880 67.031530) (end 129.307107 66.707107) (width 0.381000) (layer "F.Cu") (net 7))
 (segment (start 129.307107 66.707107) (end 128.631921 66.031921) (width 0.381000) (layer "F.Cu") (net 7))
 (arc (start 128.631921 66.031921) (mid 128.630897 66.021037) (end 128.641400 66.018000) (width 0.381000) (layer "F.Cu") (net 7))
 (segment (start 128.641400 66.018000) (end 128.692000 66.040000) (width 0.381000) (layer "F.Cu") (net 7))
 (segment (start 101.950000 69.500000) (end 106.706521 64.696385) (width 0.508000) (layer "F.Cu") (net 2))
 (arc (start 106.706521 64.696385) (mid 107.032144 64.477066) (end 107.417102 64.400000) (width 0.508000) (layer "F.Cu") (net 2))
 (segment (start 107.417102 64.400000) (end 111.153226 64.400000) (width 0.508000) (layer "F.Cu") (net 2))
 (arc (start 111.153226 64.400000) (mid 111.193737 64.410851) (end 111.223400 64.440500) (width 0.508000) (layer "F.Cu") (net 2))
 (segment (start 111.223400 64.440500) (end 111.252000 64.490000) (width 0.508000) (layer "F.Cu") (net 2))
 (segment (start 111.252000 64.490000) (end 111.223400 64.440500) (width 0.508000) (layer "F.Cu") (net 2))
 (arc (start 111.223400 64.440500) (mid 111.215746 64.402070) (end 111.233074 64.366926) (width 0.508000) (layer "F.Cu") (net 2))
 (segment (start 111.233074 64.366926) (end 112.107107 63.492893) (width 0.508000) (layer "F.Cu") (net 2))
 (arc (start 112.107107 63.492893) (mid 112.431530 63.276120) (end 112.814214 63.200000) (width 0.508000) (layer "F.Cu") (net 2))
 (segment (start 112.814214 63.200000) (end 118.763470 63.200000) (width 0.508000) (layer "F.Cu") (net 2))
 (arc (start 118.763470 63.200000) (mid 119.163543 63.283517) (end 119.496790 63.520116) (width 0.508000) (layer "F.Cu") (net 2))
 (segment (start 119.496790 63.520116) (end 120.396000 64.490000) (width 0.508000) (layer "F.Cu") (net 2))
 (segment (start 120.396000 64.490000) (end 120.508200 64.330500) (width 0.508000) (layer "F.Cu") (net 2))
 (arc (start 120.508200 64.330500) (mid 120.617948 64.234569) (end 120.759554 64.200000) (width 0.508000) (layer "F.Cu") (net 2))
 (segment (start 120.759554 64.200000) (end 122.400000 64.200000) (width 0.508000) (layer "F.Cu") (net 2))
 (segment (start 122.400000 64.200000) (end 121.892893 64.707107) (width 0.508000) (layer "B.Cu") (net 2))
 (arc (start 121.892893 64.707107) (mid 121.676120 65.031530) (end 121.600000 65.414214) (width 0.508000) (layer "B.Cu") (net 2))
 (segment (start 121.600000 65.414214) (end 121.600000 69.400000) (width 0.508000) (layer "B.Cu") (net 2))
 (segment (start 121.600000 69.400000) (end 122.725632 70.525632) (width 0.508000) (layer "F.Cu") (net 2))
 (arc (start 122.725632 70.525632) (mid 122.806313 70.589944) (end 122.899300 70.634650) (width 0.508000) (layer "F.Cu") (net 2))
 (segment (start 122.899300 70.634650) (end 123.020667 70.677000) (width 0.508000) (layer "F.Cu") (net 2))
 (segment (start 123.020667 70.677000) (end 120.630132 70.611742) (width 0.508000) (layer "F.Cu") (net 2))
 (arc (start 120.630132 70.611742) (mid 120.232803 70.682354) (end 119.895737 70.904263) (width 0.508000) (layer "F.Cu") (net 2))
 (segment (start 119.895737 70.904263) (end 119.229387 71.570613) (width 0.508000) (layer "F.Cu") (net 2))
 (arc (start 119.229387 71.570613) (mid 119.225468 71.589772) (end 119.241550 71.600900) (width 0.508000) (layer "F.Cu") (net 2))
 (segment (start 119.241550 71.600900) (end 119.292333 71.602000) (width 0.508000) (layer "F.Cu") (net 2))
 (via (at 128.400000 71.400000) (size 0.889000) (drill 0.381000) (layers "F.Cu" "B.Cu") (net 6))
 (via (at 129.600000 73.600000) (size 0.889000) (drill 0.381000) (layers "F.Cu" "B.Cu") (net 6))
 (via (at 112.400000 69.200000) (size 0.889000) (drill 0.381000) (layers "F.Cu" "B.Cu") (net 4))
 (via (at 127.600000 77.400000) (size 0.889000) (drill 0.381000) (layers "F.Cu" "B.Cu") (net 4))
 (via (at 128.400000 77.000000) (size 0.889000) (drill 0.381000) (layers "F.Cu" "B.Cu") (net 4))
 (via (at 119.200000 76.600000) (size 0.889000) (drill 0.381000) (layers "F.Cu" "B.Cu") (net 1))
 (via (at 122.000000 77.600000) (size 0.889000) (drill 0.381000) (layers "F.Cu" "B.Cu") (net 1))
 (via (at 128.400000 75.600000) (size 0.889000) (drill 0.381000) (layers "F.Cu" "B.Cu") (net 1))
 (via (at 123.000000 68.600000) (size 0.889000) (drill 0.381000) (layers "F.Cu" "B.Cu") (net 7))
 (via (at 129.600000 68.600000) (size 0.889000) (drill 0.381000) (layers "F.Cu" "B.Cu") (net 7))
 (via (at 122.400000 64.200000) (size 1.016000) (drill 0.508000) (layers "F.Cu" "B.Cu") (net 2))
 (via (at 121.600000 69.400000) (size 1.016000) (drill 0.508000) (layers "F.Cu" "B.Cu") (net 2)))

